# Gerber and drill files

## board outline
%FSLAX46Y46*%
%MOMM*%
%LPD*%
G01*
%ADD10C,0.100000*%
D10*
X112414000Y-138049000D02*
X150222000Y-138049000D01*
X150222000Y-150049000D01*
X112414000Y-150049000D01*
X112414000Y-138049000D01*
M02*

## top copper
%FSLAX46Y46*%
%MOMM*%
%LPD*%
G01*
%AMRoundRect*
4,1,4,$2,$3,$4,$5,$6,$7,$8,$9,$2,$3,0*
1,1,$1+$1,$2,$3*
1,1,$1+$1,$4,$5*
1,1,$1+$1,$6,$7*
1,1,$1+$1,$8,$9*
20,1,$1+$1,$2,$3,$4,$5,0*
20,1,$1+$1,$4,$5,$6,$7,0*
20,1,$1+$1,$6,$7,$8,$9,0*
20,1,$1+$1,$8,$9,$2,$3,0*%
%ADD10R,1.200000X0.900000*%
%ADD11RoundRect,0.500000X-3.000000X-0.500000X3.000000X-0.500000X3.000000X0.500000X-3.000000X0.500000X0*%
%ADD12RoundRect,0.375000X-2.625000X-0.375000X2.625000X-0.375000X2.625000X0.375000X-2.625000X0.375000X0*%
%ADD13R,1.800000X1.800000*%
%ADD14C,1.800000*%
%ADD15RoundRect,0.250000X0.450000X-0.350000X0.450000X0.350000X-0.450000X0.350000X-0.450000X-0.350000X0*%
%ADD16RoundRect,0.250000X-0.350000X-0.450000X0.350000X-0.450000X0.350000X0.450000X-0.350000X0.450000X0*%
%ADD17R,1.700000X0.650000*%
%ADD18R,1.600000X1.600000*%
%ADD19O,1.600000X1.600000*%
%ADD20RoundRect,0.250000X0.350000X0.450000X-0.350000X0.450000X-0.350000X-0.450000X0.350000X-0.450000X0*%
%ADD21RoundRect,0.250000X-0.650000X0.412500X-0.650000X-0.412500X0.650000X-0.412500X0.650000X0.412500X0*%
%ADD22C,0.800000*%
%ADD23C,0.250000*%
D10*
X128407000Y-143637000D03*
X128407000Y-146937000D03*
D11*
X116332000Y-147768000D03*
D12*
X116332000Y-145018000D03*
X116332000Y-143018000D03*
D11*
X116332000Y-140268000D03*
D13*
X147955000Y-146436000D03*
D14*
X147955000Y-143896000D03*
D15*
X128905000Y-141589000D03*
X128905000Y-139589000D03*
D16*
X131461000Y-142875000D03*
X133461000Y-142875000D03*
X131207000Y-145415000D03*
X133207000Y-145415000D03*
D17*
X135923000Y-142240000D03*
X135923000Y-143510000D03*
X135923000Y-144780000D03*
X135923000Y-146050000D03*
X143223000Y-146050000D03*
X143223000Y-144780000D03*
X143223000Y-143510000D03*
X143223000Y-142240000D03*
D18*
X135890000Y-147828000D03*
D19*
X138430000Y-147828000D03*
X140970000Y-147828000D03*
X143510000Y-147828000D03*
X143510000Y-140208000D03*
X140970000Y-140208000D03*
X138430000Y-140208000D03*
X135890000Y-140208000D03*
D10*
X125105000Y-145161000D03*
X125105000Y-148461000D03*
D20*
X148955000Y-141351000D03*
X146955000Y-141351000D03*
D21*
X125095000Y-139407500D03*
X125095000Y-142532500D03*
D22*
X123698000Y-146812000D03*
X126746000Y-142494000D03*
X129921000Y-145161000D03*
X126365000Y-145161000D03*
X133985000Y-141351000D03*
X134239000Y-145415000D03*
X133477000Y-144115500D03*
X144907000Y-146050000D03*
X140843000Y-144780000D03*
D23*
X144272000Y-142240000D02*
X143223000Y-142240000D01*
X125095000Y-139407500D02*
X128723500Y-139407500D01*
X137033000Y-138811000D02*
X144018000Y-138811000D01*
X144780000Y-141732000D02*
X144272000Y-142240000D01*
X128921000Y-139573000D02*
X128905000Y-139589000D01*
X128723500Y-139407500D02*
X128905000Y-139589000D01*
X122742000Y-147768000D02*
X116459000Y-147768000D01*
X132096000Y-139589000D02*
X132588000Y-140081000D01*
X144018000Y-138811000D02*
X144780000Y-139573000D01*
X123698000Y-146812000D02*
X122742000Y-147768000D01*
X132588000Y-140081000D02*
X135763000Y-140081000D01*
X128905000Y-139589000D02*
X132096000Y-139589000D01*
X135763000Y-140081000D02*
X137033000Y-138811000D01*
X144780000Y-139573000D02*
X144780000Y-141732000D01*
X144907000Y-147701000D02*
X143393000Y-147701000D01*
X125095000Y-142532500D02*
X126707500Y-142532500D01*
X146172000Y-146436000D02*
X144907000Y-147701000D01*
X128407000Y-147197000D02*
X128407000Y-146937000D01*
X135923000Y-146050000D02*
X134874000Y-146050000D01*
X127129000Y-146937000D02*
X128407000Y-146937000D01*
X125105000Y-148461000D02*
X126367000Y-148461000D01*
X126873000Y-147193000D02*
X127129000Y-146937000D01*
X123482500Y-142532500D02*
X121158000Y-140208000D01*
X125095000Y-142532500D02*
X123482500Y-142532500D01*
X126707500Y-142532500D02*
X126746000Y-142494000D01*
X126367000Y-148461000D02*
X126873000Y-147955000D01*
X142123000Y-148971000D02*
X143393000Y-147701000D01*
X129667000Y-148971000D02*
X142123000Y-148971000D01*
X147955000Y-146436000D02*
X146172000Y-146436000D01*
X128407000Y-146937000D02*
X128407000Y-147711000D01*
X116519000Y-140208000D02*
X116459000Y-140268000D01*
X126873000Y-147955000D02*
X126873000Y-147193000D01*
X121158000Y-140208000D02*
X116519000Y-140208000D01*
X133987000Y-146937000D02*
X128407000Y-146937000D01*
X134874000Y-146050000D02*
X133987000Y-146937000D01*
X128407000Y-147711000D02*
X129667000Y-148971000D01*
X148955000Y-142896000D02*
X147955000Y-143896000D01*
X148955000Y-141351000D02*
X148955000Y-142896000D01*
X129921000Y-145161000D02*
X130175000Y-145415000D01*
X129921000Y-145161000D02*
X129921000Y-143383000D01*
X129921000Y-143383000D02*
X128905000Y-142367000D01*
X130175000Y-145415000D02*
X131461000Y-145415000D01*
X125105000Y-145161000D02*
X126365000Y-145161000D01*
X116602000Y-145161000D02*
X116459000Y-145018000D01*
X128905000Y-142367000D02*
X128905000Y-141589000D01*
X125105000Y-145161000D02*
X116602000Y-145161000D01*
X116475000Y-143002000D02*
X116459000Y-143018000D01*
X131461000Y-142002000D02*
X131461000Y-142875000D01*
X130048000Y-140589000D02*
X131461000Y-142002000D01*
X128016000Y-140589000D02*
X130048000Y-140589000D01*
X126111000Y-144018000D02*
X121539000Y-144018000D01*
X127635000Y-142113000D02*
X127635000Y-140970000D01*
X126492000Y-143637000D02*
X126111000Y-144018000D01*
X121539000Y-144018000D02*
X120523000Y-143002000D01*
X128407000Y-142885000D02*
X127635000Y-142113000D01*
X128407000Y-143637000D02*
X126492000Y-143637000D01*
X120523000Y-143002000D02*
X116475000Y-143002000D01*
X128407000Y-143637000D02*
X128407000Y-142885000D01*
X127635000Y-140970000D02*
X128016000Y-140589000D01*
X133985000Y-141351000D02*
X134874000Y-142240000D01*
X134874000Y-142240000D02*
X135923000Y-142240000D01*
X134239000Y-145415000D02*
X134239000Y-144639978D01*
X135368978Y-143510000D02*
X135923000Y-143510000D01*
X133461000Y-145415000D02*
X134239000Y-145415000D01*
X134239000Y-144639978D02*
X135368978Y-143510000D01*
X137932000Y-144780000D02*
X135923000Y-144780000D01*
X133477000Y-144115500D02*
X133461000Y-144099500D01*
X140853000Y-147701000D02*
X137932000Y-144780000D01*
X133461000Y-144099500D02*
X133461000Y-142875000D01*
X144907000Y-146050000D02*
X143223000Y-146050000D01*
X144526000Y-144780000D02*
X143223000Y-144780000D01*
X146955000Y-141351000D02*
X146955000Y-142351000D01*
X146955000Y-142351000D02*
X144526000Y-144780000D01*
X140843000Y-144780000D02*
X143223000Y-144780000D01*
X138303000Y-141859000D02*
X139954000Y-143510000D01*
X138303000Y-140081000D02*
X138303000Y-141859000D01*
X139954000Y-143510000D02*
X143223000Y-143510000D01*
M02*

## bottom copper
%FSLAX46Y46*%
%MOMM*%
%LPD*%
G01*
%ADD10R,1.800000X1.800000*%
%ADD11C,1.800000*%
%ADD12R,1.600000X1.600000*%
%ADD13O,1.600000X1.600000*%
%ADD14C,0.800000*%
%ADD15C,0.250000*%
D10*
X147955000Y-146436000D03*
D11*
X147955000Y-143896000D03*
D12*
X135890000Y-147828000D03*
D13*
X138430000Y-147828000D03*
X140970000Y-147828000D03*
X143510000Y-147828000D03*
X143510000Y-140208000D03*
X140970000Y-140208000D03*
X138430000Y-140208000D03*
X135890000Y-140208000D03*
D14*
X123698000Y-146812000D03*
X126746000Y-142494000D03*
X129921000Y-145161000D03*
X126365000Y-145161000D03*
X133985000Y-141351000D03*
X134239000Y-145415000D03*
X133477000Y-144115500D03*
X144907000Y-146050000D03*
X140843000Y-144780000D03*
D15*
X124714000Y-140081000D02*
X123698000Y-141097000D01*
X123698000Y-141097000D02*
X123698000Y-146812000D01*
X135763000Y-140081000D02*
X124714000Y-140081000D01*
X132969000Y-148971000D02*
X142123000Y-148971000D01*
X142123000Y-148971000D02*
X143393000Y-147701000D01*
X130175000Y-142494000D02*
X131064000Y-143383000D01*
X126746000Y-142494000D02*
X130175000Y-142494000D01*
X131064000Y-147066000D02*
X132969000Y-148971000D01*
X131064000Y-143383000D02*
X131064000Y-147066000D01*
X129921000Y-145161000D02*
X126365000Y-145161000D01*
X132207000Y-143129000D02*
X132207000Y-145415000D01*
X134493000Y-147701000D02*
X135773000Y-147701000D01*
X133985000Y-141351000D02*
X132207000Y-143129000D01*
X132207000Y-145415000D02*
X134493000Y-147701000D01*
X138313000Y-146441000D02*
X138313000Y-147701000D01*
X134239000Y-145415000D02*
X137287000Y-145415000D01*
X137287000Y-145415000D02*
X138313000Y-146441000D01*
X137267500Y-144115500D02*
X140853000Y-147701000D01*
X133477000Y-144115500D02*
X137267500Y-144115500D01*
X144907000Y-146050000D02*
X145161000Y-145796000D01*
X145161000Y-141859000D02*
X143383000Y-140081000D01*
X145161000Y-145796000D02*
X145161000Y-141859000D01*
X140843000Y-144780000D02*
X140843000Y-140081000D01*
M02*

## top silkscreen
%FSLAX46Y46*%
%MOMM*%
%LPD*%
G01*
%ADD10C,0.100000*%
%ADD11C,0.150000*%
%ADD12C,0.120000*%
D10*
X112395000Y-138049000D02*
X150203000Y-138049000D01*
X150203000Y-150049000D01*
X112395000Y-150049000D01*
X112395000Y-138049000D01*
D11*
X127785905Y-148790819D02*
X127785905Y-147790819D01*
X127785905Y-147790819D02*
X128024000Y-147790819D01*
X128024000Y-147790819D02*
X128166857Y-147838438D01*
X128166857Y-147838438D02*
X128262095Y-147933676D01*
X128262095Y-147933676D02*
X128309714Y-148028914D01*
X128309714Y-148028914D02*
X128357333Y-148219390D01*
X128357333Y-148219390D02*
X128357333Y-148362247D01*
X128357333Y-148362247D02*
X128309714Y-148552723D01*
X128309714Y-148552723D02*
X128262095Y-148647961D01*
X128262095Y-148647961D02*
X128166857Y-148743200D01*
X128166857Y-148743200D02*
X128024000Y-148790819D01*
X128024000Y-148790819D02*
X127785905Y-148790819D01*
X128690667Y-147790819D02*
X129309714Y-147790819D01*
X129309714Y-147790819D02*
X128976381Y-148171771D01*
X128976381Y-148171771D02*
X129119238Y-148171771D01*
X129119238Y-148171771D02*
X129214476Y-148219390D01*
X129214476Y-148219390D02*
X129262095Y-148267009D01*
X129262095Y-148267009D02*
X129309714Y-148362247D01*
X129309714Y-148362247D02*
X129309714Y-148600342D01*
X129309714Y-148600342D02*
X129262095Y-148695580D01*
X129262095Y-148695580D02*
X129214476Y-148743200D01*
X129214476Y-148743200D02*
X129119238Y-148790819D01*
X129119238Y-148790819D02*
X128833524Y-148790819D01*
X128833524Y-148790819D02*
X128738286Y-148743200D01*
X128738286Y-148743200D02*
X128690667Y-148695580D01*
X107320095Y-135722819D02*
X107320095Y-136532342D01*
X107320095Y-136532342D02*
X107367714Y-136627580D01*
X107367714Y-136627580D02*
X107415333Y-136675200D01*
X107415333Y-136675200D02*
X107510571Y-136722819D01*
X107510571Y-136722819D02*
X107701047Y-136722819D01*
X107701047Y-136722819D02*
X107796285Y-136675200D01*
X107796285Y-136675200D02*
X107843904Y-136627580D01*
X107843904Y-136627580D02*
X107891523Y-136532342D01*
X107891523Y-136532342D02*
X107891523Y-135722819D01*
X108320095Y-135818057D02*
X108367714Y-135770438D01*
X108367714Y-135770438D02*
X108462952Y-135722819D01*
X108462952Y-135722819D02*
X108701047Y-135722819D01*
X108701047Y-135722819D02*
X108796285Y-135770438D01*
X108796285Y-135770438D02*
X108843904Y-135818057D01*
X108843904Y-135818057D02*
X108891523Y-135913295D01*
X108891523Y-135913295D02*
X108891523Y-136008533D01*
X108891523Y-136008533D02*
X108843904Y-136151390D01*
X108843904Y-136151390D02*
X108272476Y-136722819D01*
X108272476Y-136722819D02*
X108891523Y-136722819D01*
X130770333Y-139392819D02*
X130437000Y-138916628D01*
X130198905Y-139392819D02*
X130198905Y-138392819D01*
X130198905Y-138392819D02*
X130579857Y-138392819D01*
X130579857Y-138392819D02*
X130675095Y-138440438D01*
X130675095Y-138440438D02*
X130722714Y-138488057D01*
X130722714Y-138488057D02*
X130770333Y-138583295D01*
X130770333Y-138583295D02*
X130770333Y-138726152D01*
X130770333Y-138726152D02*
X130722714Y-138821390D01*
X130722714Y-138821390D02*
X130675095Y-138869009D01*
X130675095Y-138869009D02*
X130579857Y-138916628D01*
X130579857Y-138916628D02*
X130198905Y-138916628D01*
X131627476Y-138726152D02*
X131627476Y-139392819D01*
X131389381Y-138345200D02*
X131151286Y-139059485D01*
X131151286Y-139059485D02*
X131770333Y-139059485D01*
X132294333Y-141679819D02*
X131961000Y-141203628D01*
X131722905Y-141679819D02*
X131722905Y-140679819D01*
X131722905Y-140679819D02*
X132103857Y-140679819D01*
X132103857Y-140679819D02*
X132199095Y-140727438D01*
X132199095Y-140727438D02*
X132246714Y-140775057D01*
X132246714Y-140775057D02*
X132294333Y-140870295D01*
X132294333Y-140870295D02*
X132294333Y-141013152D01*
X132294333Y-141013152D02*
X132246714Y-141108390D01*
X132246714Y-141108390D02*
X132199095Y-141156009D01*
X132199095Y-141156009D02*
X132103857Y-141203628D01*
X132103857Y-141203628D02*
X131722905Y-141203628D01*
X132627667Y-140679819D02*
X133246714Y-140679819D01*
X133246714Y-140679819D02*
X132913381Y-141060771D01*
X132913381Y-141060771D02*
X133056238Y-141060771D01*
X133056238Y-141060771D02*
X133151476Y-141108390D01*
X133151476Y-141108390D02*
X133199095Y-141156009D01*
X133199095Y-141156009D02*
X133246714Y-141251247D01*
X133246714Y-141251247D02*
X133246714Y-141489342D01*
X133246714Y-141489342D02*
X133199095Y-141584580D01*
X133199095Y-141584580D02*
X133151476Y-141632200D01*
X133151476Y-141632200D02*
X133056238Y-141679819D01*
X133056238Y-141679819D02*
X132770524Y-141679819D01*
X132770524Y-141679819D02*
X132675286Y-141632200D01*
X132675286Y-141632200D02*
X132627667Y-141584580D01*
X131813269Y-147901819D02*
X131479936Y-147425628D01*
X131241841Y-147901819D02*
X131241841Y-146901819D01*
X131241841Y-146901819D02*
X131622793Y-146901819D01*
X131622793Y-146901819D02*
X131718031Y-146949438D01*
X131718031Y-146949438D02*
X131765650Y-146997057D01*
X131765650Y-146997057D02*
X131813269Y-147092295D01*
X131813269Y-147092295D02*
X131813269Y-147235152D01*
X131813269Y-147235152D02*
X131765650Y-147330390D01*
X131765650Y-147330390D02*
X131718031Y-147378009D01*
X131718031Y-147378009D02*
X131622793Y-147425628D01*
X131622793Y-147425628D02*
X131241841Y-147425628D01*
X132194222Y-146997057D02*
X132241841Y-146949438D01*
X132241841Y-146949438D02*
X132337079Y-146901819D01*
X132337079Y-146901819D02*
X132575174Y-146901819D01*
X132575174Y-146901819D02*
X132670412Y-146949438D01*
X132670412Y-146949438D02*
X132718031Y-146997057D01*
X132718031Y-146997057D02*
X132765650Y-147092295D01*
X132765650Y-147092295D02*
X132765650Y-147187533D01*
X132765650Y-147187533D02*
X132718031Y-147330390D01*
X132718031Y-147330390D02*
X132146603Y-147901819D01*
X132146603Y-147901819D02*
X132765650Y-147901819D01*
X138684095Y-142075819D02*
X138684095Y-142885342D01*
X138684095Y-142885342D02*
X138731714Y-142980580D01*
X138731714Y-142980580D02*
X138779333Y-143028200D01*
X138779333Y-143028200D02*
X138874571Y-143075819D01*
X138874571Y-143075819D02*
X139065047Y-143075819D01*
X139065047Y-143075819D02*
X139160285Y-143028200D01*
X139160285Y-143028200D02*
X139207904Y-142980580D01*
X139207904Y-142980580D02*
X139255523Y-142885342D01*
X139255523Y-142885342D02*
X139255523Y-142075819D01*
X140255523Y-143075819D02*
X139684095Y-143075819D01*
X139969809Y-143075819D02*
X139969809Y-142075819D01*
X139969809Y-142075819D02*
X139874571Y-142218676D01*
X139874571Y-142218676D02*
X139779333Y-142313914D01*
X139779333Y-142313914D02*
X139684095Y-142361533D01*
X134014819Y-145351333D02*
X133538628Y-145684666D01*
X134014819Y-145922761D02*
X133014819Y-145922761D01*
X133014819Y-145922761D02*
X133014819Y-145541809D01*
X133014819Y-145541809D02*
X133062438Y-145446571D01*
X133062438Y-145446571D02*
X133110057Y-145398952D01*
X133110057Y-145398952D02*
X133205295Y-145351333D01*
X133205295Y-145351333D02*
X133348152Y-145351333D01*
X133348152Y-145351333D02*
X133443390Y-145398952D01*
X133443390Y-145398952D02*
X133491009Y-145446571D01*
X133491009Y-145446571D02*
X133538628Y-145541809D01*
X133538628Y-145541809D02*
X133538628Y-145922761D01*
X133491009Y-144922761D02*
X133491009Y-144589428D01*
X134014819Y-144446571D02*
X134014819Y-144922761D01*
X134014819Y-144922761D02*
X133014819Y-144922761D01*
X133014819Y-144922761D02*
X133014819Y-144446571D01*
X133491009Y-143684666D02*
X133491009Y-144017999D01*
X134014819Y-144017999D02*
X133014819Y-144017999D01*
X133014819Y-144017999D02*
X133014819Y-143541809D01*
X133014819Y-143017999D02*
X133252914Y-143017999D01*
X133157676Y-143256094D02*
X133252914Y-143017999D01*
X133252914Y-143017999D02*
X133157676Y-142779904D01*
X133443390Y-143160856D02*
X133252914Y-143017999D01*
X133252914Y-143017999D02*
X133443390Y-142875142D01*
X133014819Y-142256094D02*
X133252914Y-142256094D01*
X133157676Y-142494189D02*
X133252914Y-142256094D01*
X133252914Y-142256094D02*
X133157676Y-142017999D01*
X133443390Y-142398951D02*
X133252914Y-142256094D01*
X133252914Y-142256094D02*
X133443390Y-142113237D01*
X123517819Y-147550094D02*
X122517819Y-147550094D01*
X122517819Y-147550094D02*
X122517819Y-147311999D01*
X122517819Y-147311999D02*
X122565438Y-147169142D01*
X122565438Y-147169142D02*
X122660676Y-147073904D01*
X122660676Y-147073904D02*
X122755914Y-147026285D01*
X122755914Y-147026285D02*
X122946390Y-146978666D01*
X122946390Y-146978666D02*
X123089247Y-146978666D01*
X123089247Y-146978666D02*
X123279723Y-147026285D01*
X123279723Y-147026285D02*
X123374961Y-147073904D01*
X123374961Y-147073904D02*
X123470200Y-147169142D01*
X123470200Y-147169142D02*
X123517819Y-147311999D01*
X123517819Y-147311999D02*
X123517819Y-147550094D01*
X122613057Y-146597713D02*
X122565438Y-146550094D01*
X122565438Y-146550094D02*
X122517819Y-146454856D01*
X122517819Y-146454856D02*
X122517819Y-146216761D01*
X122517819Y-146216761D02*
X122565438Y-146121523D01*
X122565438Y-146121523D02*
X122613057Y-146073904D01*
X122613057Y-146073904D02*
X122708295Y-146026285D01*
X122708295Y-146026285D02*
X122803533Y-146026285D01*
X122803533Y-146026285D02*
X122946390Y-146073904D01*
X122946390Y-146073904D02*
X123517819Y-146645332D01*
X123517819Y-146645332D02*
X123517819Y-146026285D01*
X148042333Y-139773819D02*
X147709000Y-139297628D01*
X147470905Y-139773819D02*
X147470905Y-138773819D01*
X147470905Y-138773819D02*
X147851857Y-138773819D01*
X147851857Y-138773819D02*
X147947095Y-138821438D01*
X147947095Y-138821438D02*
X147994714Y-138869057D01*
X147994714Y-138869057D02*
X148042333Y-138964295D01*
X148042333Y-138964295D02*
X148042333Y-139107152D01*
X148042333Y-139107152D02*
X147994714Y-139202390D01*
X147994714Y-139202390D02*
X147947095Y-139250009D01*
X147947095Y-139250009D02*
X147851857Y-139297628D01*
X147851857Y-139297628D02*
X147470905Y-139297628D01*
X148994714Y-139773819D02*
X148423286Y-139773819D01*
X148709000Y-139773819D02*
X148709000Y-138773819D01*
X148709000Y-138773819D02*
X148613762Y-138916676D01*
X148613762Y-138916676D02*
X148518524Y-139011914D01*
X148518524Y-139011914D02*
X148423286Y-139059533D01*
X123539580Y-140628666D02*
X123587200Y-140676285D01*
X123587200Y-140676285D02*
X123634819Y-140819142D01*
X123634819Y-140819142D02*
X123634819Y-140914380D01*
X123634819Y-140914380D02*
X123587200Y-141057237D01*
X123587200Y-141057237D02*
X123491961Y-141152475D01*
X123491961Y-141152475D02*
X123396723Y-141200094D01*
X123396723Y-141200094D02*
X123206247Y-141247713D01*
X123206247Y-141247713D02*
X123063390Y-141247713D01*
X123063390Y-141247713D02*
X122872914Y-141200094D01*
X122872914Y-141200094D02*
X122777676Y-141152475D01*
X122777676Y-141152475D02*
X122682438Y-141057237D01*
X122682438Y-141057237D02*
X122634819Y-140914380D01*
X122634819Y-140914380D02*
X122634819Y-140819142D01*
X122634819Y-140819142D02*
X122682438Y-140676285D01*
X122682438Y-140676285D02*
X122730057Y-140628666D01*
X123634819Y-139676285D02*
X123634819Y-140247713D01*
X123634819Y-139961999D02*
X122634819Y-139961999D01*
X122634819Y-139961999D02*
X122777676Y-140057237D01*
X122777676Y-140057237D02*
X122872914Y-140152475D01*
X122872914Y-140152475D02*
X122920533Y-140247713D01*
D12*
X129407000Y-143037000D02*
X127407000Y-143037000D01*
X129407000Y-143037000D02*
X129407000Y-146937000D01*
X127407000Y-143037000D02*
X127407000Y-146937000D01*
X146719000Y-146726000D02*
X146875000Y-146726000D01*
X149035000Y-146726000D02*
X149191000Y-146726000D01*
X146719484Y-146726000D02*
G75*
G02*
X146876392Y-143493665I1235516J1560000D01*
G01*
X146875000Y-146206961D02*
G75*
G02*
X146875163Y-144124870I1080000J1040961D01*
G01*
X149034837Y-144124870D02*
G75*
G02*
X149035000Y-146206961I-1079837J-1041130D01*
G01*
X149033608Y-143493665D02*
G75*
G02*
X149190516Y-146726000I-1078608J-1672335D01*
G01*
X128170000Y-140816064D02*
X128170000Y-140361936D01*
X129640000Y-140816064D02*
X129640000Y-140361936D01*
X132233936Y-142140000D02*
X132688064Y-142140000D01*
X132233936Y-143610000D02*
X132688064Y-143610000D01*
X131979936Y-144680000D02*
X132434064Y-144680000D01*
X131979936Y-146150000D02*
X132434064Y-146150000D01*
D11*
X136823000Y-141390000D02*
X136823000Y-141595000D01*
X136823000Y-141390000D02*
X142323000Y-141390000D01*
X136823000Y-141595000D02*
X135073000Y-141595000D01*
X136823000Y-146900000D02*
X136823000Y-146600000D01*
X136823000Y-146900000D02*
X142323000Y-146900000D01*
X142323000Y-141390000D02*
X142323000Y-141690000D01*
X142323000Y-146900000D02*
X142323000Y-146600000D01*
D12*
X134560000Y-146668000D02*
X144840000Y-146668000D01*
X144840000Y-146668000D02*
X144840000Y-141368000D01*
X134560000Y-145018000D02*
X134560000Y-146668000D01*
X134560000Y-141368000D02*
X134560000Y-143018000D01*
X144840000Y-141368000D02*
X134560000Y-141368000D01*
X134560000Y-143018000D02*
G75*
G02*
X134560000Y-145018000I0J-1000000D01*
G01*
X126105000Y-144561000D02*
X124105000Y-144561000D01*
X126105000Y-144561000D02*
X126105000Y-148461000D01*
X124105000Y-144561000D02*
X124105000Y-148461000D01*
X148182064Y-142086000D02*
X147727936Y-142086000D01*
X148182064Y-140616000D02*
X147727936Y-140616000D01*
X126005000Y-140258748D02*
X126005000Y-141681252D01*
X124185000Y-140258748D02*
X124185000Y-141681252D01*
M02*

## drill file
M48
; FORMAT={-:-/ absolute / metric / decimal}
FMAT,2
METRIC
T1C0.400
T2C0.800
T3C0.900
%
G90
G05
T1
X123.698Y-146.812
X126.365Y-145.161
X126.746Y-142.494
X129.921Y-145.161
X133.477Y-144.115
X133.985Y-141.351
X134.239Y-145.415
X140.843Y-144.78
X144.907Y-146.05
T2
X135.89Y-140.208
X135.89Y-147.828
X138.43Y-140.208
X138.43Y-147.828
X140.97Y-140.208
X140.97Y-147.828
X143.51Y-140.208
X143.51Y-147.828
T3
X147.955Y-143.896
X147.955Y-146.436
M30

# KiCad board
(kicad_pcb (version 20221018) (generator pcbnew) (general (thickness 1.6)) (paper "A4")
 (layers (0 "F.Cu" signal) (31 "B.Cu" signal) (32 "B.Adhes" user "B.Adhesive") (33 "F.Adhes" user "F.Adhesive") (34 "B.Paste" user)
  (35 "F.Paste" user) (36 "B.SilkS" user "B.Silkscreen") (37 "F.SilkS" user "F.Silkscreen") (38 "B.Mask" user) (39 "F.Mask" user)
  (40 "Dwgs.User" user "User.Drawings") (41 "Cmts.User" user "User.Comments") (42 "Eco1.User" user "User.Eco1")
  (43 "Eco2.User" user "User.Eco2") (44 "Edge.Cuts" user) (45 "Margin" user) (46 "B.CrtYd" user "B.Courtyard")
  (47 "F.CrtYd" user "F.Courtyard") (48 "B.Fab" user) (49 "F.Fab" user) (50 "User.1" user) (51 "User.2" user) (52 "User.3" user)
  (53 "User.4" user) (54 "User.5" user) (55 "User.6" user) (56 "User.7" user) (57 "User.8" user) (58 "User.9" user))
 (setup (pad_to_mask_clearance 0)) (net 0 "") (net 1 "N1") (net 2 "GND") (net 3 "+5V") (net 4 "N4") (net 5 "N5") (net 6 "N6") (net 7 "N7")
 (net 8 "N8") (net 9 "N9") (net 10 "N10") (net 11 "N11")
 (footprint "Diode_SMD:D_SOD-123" (layer "F.Cu") (at 128.407 145.287 -90)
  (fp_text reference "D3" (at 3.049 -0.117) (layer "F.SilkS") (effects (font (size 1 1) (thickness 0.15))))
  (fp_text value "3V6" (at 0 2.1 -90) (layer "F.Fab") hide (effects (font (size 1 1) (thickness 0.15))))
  (fp_line (start -2.25 -1) (end -2.25 1) (stroke (width 0.12) (type solid)) (layer "F.SilkS"))
  (fp_line (start -2.25 -1) (end 1.65 -1) (stroke (width 0.12) (type solid)) (layer "F.SilkS"))
  (fp_line (start -2.25 1) (end 1.65 1) (stroke (width 0.12) (type solid)) (layer "F.SilkS"))
  (pad "1" smd rect (at -1.65 0 270) (size 0.9 1.2) (layers "F.Cu" "F.Paste" "F.Mask") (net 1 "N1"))
  (pad "2" smd rect (at 1.65 0 270) (size 0.9 1.2) (layers "F.Cu" "F.Paste" "F.Mask") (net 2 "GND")))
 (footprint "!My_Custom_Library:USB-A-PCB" (layer "F.Cu") (at 116.332 144.018)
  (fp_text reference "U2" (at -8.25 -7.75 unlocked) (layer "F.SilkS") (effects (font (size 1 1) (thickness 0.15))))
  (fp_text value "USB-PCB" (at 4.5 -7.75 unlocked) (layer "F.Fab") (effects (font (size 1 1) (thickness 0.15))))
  (pad "1" smd roundrect (at 0 3.75) (size 7 2) (layers "F.Cu" "F.Paste" "F.Mask") (roundrect_rratio 0.25) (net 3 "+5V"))
  (pad "2" smd roundrect (at 0 1) (size 6 1.5) (layers "F.Cu" "F.Paste" "F.Mask") (roundrect_rratio 0.25) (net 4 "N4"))
  (pad "3" smd roundrect (at 0 -1) (size 6 1.5) (layers "F.Cu" "F.Paste" "F.Mask") (roundrect_rratio 0.25) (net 1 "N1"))
  (pad "4" smd roundrect (at 0 -3.75) (size 7 2) (layers "F.Cu" "F.Paste" "F.Mask") (roundrect_rratio 0.25) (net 2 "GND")))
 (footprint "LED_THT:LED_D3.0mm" (layer "F.Cu") (at 147.955 146.436 90)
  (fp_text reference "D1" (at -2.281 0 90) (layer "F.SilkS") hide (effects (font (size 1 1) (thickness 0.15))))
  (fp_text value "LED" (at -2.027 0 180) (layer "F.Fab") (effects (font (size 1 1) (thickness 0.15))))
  (fp_line (start -0.29 -1.236) (end -0.29 -1.08) (stroke (width 0.12) (type solid)) (layer "F.SilkS"))
  (fp_line (start -0.29 1.08) (end -0.29 1.236) (stroke (width 0.12) (type solid)) (layer "F.SilkS"))
  (fp_arc (start -0.29 -1.235516) (mid 1.366487 -1.987659) (end 2.942335 -1.078608) (stroke (width 0.12) (type solid)) (layer "F.SilkS"))
  (fp_arc (start 0.229039 -1.08) (mid 1.270117 -1.5) (end 2.31113 -1.079837) (stroke (width 0.12) (type solid)) (layer "F.SilkS"))
  (fp_arc (start 2.31113 1.079837) (mid 1.270117 1.5) (end 0.229039 1.08) (stroke (width 0.12) (type solid)) (layer "F.SilkS"))
  (fp_arc (start 2.942335 1.078608) (mid 1.366487 1.987659) (end -0.29 1.235516) (stroke (width 0.12) (type solid)) (layer "F.SilkS"))
  (pad "1" thru_hole rect (at 0 0 90) (size 1.8 1.8) (drill 0.9) (layers "*.Cu" "*.Mask") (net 2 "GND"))
  (pad "2" thru_hole circle (at 2.54 0 90) (size 1.8 1.8) (drill 0.9) (layers "*.Cu" "*.Mask") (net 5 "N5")))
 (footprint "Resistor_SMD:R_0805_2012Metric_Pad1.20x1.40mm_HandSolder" (layer "F.Cu") (at 128.905 140.589 90)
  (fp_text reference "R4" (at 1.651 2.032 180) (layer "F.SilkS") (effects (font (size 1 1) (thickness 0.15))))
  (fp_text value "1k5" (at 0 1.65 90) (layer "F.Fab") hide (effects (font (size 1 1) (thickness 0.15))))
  (fp_line (start -0.227064 -0.735) (end 0.227064 -0.735) (stroke (width 0.12) (type solid)) (layer "F.SilkS"))
  (fp_line (start -0.227064 0.735) (end 0.227064 0.735) (stroke (width 0.12) (type solid)) (layer "F.SilkS"))
  (pad "1" smd roundrect (at -1 0 90) (size 1.2 1.4) (layers "F.Cu" "F.Paste" "F.Mask") (roundrect_rratio 0.2083333333) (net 4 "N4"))
  (pad "2" smd roundrect (at 1 0 90) (size 1.2 1.4) (layers "F.Cu" "F.Paste" "F.Mask") (roundrect_rratio 0.2083333333) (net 3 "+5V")))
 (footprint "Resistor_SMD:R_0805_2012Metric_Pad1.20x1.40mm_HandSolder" (layer "F.Cu") (at 132.461 142.875)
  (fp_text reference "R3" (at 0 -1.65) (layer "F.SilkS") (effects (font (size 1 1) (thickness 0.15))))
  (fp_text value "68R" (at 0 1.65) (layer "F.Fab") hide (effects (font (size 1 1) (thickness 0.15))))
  (fp_line (start -0.227064 -0.735) (end 0.227064 -0.735) (stroke (width 0.12) (type solid)) (layer "F.SilkS"))
  (fp_line (start -0.227064 0.735) (end 0.227064 0.735) (stroke (width 0.12) (type solid)) (layer "F.SilkS"))
  (pad "1" smd roundrect (at -1 0) (size 1.2 1.4) (layers "F.Cu" "F.Paste" "F.Mask") (roundrect_rratio 0.2083333333) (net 1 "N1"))
  (pad "2" smd roundrect (at 1 0) (size 1.2 1.4) (layers "F.Cu" "F.Paste" "F.Mask") (roundrect_rratio 0.2083333333) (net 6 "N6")))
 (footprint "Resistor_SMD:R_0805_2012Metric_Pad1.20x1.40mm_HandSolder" (layer "F.Cu") (at 132.207 145.415)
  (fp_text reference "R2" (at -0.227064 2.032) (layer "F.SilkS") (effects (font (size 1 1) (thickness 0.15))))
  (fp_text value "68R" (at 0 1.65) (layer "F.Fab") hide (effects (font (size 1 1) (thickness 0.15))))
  (fp_line (start -0.227064 -0.735) (end 0.227064 -0.735) (stroke (width 0.12) (type solid)) (layer "F.SilkS"))
  (fp_line (start -0.227064 0.735) (end 0.227064 0.735) (stroke (width 0.12) (type solid)) (layer "F.SilkS"))
  (pad "1" smd roundrect (at -1 0) (size 1.2 1.4) (layers "F.Cu" "F.Paste" "F.Mask") (roundrect_rratio 0.2083333333) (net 4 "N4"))
  (pad "2" smd roundrect (at 1 0) (size 1.2 1.4) (layers "F.Cu" "F.Paste" "F.Mask") (roundrect_rratio 0.2083333333) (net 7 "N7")))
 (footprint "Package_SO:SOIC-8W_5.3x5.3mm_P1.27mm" (layer "F.Cu") (at 139.573 144.145)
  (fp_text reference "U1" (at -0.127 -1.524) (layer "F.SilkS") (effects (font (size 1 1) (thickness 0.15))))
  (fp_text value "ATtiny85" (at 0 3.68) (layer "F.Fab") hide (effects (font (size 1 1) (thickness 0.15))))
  (fp_line (start -2.75 -2.755) (end -2.75 -2.55) (stroke (width 0.15) (type solid)) (layer "F.SilkS"))
  (fp_line (start -2.75 -2.755) (end 2.75 -2.755) (stroke (width 0.15) (type solid)) (layer "F.SilkS"))
  (fp_line (start -2.75 -2.55) (end -4.5 -2.55) (stroke (width 0.15) (type solid)) (layer "F.SilkS"))
  (fp_line (start -2.75 2.755) (end -2.75 2.455) (stroke (width 0.15) (type solid)) (layer "F.SilkS"))
  (fp_line (start -2.75 2.755) (end 2.75 2.755) (stroke (width 0.15) (type solid)) (layer "F.SilkS"))
  (fp_line (start 2.75 -2.755) (end 2.75 -2.455) (stroke (width 0.15) (type solid)) (layer "F.SilkS"))
  (fp_line (start 2.75 2.755) (end 2.75 2.455) (stroke (width 0.15) (type solid)) (layer "F.SilkS"))
  (pad "1" smd rect (at -3.65 -1.905) (size 1.7 0.65) (layers "F.Cu" "F.Paste" "F.Mask") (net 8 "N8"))
  (pad "2" smd rect (at -3.65 -0.635) (size 1.7 0.65) (layers "F.Cu" "F.Paste" "F.Mask") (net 7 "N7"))
  (pad "3" smd rect (at -3.65 0.635) (size 1.7 0.65) (layers "F.Cu" "F.Paste" "F.Mask") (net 6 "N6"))
  (pad "4" smd rect (at -3.65 1.905) (size 1.7 0.65) (layers "F.Cu" "F.Paste" "F.Mask") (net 2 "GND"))
  (pad "5" smd rect (at 3.65 1.905) (size 1.7 0.65) (layers "F.Cu" "F.Paste" "F.Mask") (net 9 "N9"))
  (pad "6" smd rect (at 3.65 0.635) (size 1.7 0.65) (layers "F.Cu" "F.Paste" "F.Mask") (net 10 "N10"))
  (pad "7" smd rect (at 3.65 -0.635) (size 1.7 0.65) (layers "F.Cu" "F.Paste" "F.Mask") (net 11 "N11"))
  (pad "8" smd rect (at 3.65 -1.905) (size 1.7 0.65) (layers "F.Cu" "F.Paste" "F.Mask") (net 3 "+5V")))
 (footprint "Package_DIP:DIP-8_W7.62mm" (layer "F.Cu") (at 135.89 147.828 90)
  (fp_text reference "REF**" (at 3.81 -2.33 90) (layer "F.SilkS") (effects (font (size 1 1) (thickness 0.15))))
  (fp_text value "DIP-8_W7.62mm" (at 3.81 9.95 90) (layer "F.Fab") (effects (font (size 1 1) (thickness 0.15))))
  (fp_line (start 1.16 -1.33) (end 1.16 8.95) (stroke (width 0.12) (type solid)) (layer "F.SilkS"))
  (fp_line (start 1.16 8.95) (end 6.46 8.95) (stroke (width 0.12) (type solid)) (layer "F.SilkS"))
  (fp_line (start 2.81 -1.33) (end 1.16 -1.33) (stroke (width 0.12) (type solid)) (layer "F.SilkS"))
  (fp_line (start 6.46 -1.33) (end 4.81 -1.33) (stroke (width 0.12) (type solid)) (layer "F.SilkS"))
  (fp_line (start 6.46 8.95) (end 6.46 -1.33) (stroke (width 0.12) (type solid)) (layer "F.SilkS"))
  (fp_arc (start 4.81 -1.33) (mid 3.81 -0.33) (end 2.81 -1.33) (stroke (width 0.12) (type solid)) (layer "F.SilkS"))
  (pad "1" thru_hole rect (at 0 0 90) (size 1.6 1.6) (drill 0.8) (layers "*.Cu" "*.Mask"))
  (pad "2" thru_hole oval (at 0 2.54 90) (size 1.6 1.6) (drill 0.8) (layers "*.Cu" "*.Mask"))
  (pad "3" thru_hole oval (at 0 5.08 90) (size 1.6 1.6) (drill 0.8) (layers "*.Cu" "*.Mask"))
  (pad "4" thru_hole oval (at 0 7.62 90) (size 1.6 1.6) (drill 0.8) (layers "*.Cu" "*.Mask"))
  (pad "5" thru_hole oval (at 7.62 7.62 90) (size 1.6 1.6) (drill 0.8) (layers "*.Cu" "*.Mask"))
  (pad "6" thru_hole oval (at 7.62 5.08 90) (size 1.6 1.6) (drill 0.8) (layers "*.Cu" "*.Mask"))
  (pad "7" thru_hole oval (at 7.62 2.54 90) (size 1.6 1.6) (drill 0.8) (layers "*.Cu" "*.Mask"))
  (pad "8" thru_hole oval (at 7.62 0 90) (size 1.6 1.6) (drill 0.8) (layers "*.Cu" "*.Mask")))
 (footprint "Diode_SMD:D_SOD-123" (layer "F.Cu") (at 125.105 146.811 -90)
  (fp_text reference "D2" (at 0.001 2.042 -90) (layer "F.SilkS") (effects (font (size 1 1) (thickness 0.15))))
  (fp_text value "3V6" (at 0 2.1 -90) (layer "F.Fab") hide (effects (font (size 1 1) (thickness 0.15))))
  (fp_line (start -2.25 -1) (end -2.25 1) (stroke (width 0.12) (type solid)) (layer "F.SilkS"))
  (fp_line (start -2.25 -1) (end 1.65 -1) (stroke (width 0.12) (type solid)) (layer "F.SilkS"))
  (fp_line (start -2.25 1) (end 1.65 1) (stroke (width 0.12) (type solid)) (layer "F.SilkS"))
  (pad "1" smd rect (at -1.65 0 270) (size 0.9 1.2) (layers "F.Cu" "F.Paste" "F.Mask") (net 4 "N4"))
  (pad "2" smd rect (at 1.65 0 270) (size 0.9 1.2) (layers "F.Cu" "F.Paste" "F.Mask") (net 2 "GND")))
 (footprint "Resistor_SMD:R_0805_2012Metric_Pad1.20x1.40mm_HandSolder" (layer "F.Cu") (at 147.955 141.351 180)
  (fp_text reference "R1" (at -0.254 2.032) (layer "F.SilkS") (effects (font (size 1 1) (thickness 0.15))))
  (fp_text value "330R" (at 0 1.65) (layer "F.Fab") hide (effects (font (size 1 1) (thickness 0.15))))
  (fp_line (start -0.227064 -0.735) (end 0.227064 -0.735) (stroke (width 0.12) (type solid)) (layer "F.SilkS"))
  (fp_line (start -0.227064 0.735) (end 0.227064 0.735) (stroke (width 0.12) (type solid)) (layer "F.SilkS"))
  (pad "1" smd roundrect (at -1 0 180) (size 1.2 1.4) (layers "F.Cu" "F.Paste" "F.Mask") (roundrect_rratio 0.2083333333) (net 5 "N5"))
  (pad "2" smd roundrect (at 1 0 180) (size 1.2 1.4) (layers "F.Cu" "F.Paste" "F.Mask") (roundrect_rratio 0.2083333333) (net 10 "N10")))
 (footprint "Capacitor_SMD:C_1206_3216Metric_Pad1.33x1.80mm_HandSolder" (layer "F.Cu") (at 125.095 140.97 -90)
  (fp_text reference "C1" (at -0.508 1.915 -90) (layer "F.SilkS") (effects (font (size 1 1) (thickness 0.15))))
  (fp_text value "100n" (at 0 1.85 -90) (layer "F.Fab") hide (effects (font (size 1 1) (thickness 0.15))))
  (fp_line (start -0.711252 -0.91) (end 0.711252 -0.91) (stroke (width 0.12) (type solid)) (layer "F.SilkS"))
  (fp_line (start -0.711252 0.91) (end 0.711252 0.91) (stroke (width 0.12) (type solid)) (layer "F.SilkS"))
  (pad "1" smd roundrect (at -1.5625 0 270) (size 1.325 1.8) (layers "F.Cu" "F.Paste" "F.Mask") (roundrect_rratio 0.1886792453)
   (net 3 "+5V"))
  (pad "2" smd roundrect (at 1.5625 0 270) (size 1.325 1.8) (layers "F.Cu" "F.Paste" "F.Mask") (roundrect_rratio 0.1886792453) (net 2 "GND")))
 (gr_rect (start 112.395 138.049) (end 150.203 150.049) (stroke (width 0.1) (type solid)) (fill none) (layer "F.SilkS"))
 (gr_rect (start 112.414 138.049) (end 150.222 150.049) (stroke (width 0.1) (type solid)) (fill none) (layer "Edge.Cuts"))
 (segment (start 144.272 142.24) (end 143.223 142.24) (width 0.25) (layer "F.Cu") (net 3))
 (segment (start 125.095 139.4075) (end 128.7235 139.4075) (width 0.25) (layer "F.Cu") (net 3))
 (segment (start 137.033 138.811) (end 144.018 138.811) (width 0.25) (layer "F.Cu") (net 3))
 (segment (start 144.78 141.732) (end 144.272 142.24) (width 0.25) (layer "F.Cu") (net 3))
 (segment (start 128.921 139.573) (end 128.905 139.589) (width 0.25) (layer "F.Cu") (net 3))
 (segment (start 128.7235 139.4075) (end 128.905 139.589) (width 0.25) (layer "F.Cu") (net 3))
 (segment (start 122.742 147.768) (end 116.459 147.768) (width 0.25) (layer "F.Cu") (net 3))
 (segment (start 132.096 139.589) (end 132.588 140.081) (width 0.25) (layer "F.Cu") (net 3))
 (segment (start 144.018 138.811) (end 144.78 139.573) (width 0.25) (layer "F.Cu") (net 3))
 (segment (start 123.698 146.812) (end 122.742 147.768) (width 0.25) (layer "F.Cu") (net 3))
 (segment (start 132.588 140.081) (end 135.763 140.081) (width 0.25) (layer "F.Cu") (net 3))
 (segment (start 128.905 139.589) (end 132.096 139.589) (width 0.25) (layer "F.Cu") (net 3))
 (segment (start 135.763 140.081) (end 137.033 138.811) (width 0.25) (layer "F.Cu") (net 3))
 (segment (start 144.78 139.573) (end 144.78 141.732) (width 0.25) (layer "F.Cu") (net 3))
 (via (at 123.698 146.812) (size 0.8) (drill 0.4) (layers "F.Cu" "B.Cu") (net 3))
 (segment (start 124.714 140.081) (end 123.698 141.097) (width 0.25) (layer "B.Cu") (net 3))
 (segment (start 123.698 141.097) (end 123.698 146.812) (width 0.25) (layer "B.Cu") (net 3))
 (segment (start 135.763 140.081) (end 124.714 140.081) (width 0.25) (layer "B.Cu") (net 3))
 (segment (start 144.907 147.701) (end 143.393 147.701) (width 0.25) (layer "F.Cu") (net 2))
 (segment (start 125.095 142.5325) (end 126.7075 142.5325) (width 0.25) (layer "F.Cu") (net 2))
 (segment (start 146.172 146.436) (end 144.907 147.701) (width 0.25) (layer "F.Cu") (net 2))
 (segment (start 128.407 147.197) (end 128.407 146.937) (width 0.25) (layer "F.Cu") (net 2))
 (segment (start 135.923 146.05) (end 134.874 146.05) (width 0.25) (layer "F.Cu") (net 2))
 (segment (start 127.129 146.937) (end 128.407 146.937) (width 0.25) (layer "F.Cu") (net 2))
 (segment (start 125.105 148.461) (end 126.367 148.461) (width 0.25) (layer "F.Cu") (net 2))
 (segment (start 126.873 147.193) (end 127.129 146.937) (width 0.25) (layer "F.Cu") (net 2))
 (segment (start 123.4825 142.5325) (end 121.158 140.208) (width 0.25) (layer "F.Cu") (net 2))
 (segment (start 125.095 142.5325) (end 123.4825 142.5325) (width 0.25) (layer "F.Cu") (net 2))
 (segment (start 126.7075 142.5325) (end 126.746 142.494) (width 0.25) (layer "F.Cu") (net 2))
 (segment (start 126.367 148.461) (end 126.873 147.955) (width 0.25) (layer "F.Cu") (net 2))
 (segment (start 142.123 148.971) (end 143.393 147.701) (width 0.25) (layer "F.Cu") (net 2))
 (segment (start 129.667 148.971) (end 142.123 148.971) (width 0.25) (layer "F.Cu") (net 2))
 (segment (start 147.955 146.436) (end 146.172 146.436) (width 0.25) (layer "F.Cu") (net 2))
 (segment (start 128.407 146.937) (end 128.407 147.711) (width 0.25) (layer "F.Cu") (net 2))
 (segment (start 116.519 140.208) (end 116.459 140.268) (width 0.25) (layer "F.Cu") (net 2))
 (segment (start 126.873 147.955) (end 126.873 147.193) (width 0.25) (layer "F.Cu") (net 2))
 (segment (start 121.158 140.208) (end 116.519 140.208) (width 0.25) (layer "F.Cu") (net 2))
 (segment (start 133.987 146.937) (end 128.407 146.937) (width 0.25) (layer "F.Cu") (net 2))
 (segment (start 134.874 146.05) (end 133.987 146.937) (width 0.25) (layer "F.Cu") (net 2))
 (segment (start 128.407 147.711) (end 129.667 148.971) (width 0.25) (layer "F.Cu") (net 2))
 (via (at 126.746 142.494) (size 0.8) (drill 0.4) (layers "F.Cu" "B.Cu") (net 2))
 (segment (start 132.969 148.971) (end 142.123 148.971) (width 0.25) (layer "B.Cu") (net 2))
 (segment (start 142.123 148.971) (end 143.393 147.701) (width 0.25) (layer "B.Cu") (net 2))
 (segment (start 130.175 142.494) (end 131.064 143.383) (width 0.25) (layer "B.Cu") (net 2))
 (segment (start 126.746 142.494) (end 130.175 142.494) (width 0.25) (layer "B.Cu") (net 2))
 (segment (start 131.064 147.066) (end 132.969 148.971) (width 0.25) (layer "B.Cu") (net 2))
 (segment (start 131.064 143.383) (end 131.064 147.066) (width 0.25) (layer "B.Cu") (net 2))
 (segment (start 148.955 142.896) (end 147.955 143.896) (width 0.25) (layer "F.Cu") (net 5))
 (segment (start 148.955 141.351) (end 148.955 142.896) (width 0.25) (layer "F.Cu") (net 5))
 (segment (start 129.921 145.161) (end 130.175 145.415) (width 0.25) (layer "F.Cu") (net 4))
 (segment (start 129.921 145.161) (end 129.921 143.383) (width 0.25) (layer "F.Cu") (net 4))
 (segment (start 129.921 143.383) (end 128.905 142.367) (width 0.25) (layer "F.Cu") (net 4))
 (segment (start 130.175 145.415) (end 131.461 145.415) (width 0.25) (layer "F.Cu") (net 4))
 (segment (start 125.105 145.161) (end 126.365 145.161) (width 0.25) (layer "F.Cu") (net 4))
 (segment (start 116.602 145.161) (end 116.459 145.018) (width 0.25) (layer "F.Cu") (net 4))
 (segment (start 128.905 142.367) (end 128.905 141.589) (width 0.25) (layer "F.Cu") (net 4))
 (segment (start 125.105 145.161) (end 116.602 145.161) (width 0.25) (layer "F.Cu") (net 4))
 (via (at 129.921 145.161) (size 0.8) (drill 0.4) (layers "F.Cu" "B.Cu") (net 4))
 (via (at 126.365 145.161) (size 0.8) (drill 0.4) (layers "F.Cu" "B.Cu") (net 4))
 (segment (start 129.921 145.161) (end 126.365 145.161) (width 0.25) (layer "B.Cu") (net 4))
 (segment (start 116.475 143.002) (end 116.459 143.018) (width 0.25) (layer "F.Cu") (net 1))
 (segment (start 131.461 142.002) (end 131.461 142.875) (width 0.25) (layer "F.Cu") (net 1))
 (segment (start 130.048 140.589) (end 131.461 142.002) (width 0.25) (layer "F.Cu") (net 1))
 (segment (start 128.016 140.589) (end 130.048 140.589) (width 0.25) (layer "F.Cu") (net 1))
 (segment (start 126.111 144.018) (end 121.539 144.018) (width 0.25) (layer "F.Cu") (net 1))
 (segment (start 127.635 142.113) (end 127.635 140.97) (width 0.25) (layer "F.Cu") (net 1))
 (segment (start 126.492 143.637) (end 126.111 144.018) (width 0.25) (layer "F.Cu") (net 1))
 (segment (start 121.539 144.018) (end 120.523 143.002) (width 0.25) (layer "F.Cu") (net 1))
 (segment (start 128.407 142.885) (end 127.635 142.113) (width 0.25) (layer "F.Cu") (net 1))
 (segment (start 128.407 143.637) (end 126.492 143.637) (width 0.25) (layer "F.Cu") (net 1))
 (segment (start 120.523 143.002) (end 116.475 143.002) (width 0.25) (layer "F.Cu") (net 1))
 (segment (start 128.407 143.637) (end 128.407 142.885) (width 0.25) (layer "F.Cu") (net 1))
 (segment (start 127.635 140.97) (end 128.016 140.589) (width 0.25) (layer "F.Cu") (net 1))
 (segment (start 133.985 141.351) (end 134.874 142.24) (width 0.25) (layer "F.Cu") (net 8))
 (segment (start 134.874 142.24) (end 135.923 142.24) (width 0.25) (layer "F.Cu") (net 8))
 (via (at 133.985 141.351) (size 0.8) (drill 0.4) (layers "F.Cu" "B.Cu") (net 8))
 (segment (start 132.207 143.129) (end 132.207 145.415) (width 0.25) (layer "B.Cu") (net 8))
 (segment (start 134.493 147.701) (end 135.773 147.701) (width 0.25) (layer "B.Cu") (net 8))
 (segment (start 133.985 141.351) (end 132.207 143.129) (width 0.25) (layer "B.Cu") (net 8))
 (segment (start 132.207 145.415) (end 134.493 147.701) (width 0.25) (layer "B.Cu") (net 8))
 (segment (start 134.239 145.415) (end 134.239 144.639978) (width 0.25) (layer "F.Cu") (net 7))
 (segment (start 135.368978 143.51) (end 135.923 143.51) (width 0.25) (layer "F.Cu") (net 7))
 (segment (start 133.461 145.415) (end 134.239 145.415) (width 0.25) (layer "F.Cu") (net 7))
 (segment (start 134.239 144.639978) (end 135.368978 143.51) (width 0.25) (layer "F.Cu") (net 7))
 (via (at 134.239 145.415) (size 0.8) (drill 0.4) (layers "F.Cu" "B.Cu") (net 7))
 (segment (start 138.313 146.441) (end 138.313 147.701) (width 0.25) (layer "B.Cu") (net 7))
 (segment (start 134.239 145.415) (end 137.287 145.415) (width 0.25) (layer "B.Cu") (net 7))
 (segment (start 137.287 145.415) (end 138.313 146.441) (width 0.25) (layer "B.Cu") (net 7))
 (segment (start 137.932 144.78) (end 135.923 144.78) (width 0.25) (layer "F.Cu") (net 6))
 (segment (start 133.477 144.1155) (end 133.461 144.0995) (width 0.25) (layer "F.Cu") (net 6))
 (segment (start 140.853 147.701) (end 137.932 144.78) (width 0.25) (layer "F.Cu") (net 6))
 (segment (start 133.461 144.0995) (end 133.461 142.875) (width 0.25) (layer "F.Cu") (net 6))
 (via (at 133.477 144.1155) (size 0.8) (drill 0.4) (layers "F.Cu" "B.Cu") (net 6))
 (segment (start 137.2675 144.1155) (end 140.853 147.701) (width 0.25) (layer "B.Cu") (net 6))
 (segment (start 133.477 144.1155) (end 137.2675 144.1155) (width 0.25) (layer "B.Cu") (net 6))
 (segment (start 144.907 146.05) (end 143.223 146.05) (width 0.25) (layer "F.Cu") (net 9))
 (via (at 144.907 146.05) (size 0.8) (drill 0.4) (layers "F.Cu" "B.Cu") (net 9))
 (segment (start 144.907 146.05) (end 145.161 145.796) (width 0.25) (layer "B.Cu") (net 9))
 (segment (start 145.161 141.859) (end 143.383 140.081) (width 0.25) (layer "B.Cu") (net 9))
 (segment (start 145.161 145.796) (end 145.161 141.859) (width 0.25) (layer "B.Cu") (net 9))
 (segment (start 144.526 144.78) (end 143.223 144.78) (width 0.25) (layer "F.Cu") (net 10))
 (segment (start 146.955 141.351) (end 146.955 142.351) (width 0.25) (layer "F.Cu") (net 10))
 (segment (start 146.955 142.351) (end 144.526 144.78) (width 0.25) (layer "F.Cu") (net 10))
 (segment (start 140.843 144.78) (end 143.223 144.78) (width 0.25) (layer "F.Cu") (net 10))
 (via (at 140.843 144.78) (size 0.8) (drill 0.4) (layers "F.Cu" "B.Cu") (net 10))
 (segment (start 140.843 144.78) (end 140.843 140.081) (width 0.25) (layer "B.Cu") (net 10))
 (segment (start 138.303 141.859) (end 139.954 143.51) (width 0.25) (layer "F.Cu") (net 11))
 (segment (start 138.303 140.081) (end 138.303 141.859) (width 0.25) (layer "F.Cu") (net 11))
 (segment (start 139.954 143.51) (end 143.223 143.51) (width 0.25) (layer "F.Cu") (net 11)))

